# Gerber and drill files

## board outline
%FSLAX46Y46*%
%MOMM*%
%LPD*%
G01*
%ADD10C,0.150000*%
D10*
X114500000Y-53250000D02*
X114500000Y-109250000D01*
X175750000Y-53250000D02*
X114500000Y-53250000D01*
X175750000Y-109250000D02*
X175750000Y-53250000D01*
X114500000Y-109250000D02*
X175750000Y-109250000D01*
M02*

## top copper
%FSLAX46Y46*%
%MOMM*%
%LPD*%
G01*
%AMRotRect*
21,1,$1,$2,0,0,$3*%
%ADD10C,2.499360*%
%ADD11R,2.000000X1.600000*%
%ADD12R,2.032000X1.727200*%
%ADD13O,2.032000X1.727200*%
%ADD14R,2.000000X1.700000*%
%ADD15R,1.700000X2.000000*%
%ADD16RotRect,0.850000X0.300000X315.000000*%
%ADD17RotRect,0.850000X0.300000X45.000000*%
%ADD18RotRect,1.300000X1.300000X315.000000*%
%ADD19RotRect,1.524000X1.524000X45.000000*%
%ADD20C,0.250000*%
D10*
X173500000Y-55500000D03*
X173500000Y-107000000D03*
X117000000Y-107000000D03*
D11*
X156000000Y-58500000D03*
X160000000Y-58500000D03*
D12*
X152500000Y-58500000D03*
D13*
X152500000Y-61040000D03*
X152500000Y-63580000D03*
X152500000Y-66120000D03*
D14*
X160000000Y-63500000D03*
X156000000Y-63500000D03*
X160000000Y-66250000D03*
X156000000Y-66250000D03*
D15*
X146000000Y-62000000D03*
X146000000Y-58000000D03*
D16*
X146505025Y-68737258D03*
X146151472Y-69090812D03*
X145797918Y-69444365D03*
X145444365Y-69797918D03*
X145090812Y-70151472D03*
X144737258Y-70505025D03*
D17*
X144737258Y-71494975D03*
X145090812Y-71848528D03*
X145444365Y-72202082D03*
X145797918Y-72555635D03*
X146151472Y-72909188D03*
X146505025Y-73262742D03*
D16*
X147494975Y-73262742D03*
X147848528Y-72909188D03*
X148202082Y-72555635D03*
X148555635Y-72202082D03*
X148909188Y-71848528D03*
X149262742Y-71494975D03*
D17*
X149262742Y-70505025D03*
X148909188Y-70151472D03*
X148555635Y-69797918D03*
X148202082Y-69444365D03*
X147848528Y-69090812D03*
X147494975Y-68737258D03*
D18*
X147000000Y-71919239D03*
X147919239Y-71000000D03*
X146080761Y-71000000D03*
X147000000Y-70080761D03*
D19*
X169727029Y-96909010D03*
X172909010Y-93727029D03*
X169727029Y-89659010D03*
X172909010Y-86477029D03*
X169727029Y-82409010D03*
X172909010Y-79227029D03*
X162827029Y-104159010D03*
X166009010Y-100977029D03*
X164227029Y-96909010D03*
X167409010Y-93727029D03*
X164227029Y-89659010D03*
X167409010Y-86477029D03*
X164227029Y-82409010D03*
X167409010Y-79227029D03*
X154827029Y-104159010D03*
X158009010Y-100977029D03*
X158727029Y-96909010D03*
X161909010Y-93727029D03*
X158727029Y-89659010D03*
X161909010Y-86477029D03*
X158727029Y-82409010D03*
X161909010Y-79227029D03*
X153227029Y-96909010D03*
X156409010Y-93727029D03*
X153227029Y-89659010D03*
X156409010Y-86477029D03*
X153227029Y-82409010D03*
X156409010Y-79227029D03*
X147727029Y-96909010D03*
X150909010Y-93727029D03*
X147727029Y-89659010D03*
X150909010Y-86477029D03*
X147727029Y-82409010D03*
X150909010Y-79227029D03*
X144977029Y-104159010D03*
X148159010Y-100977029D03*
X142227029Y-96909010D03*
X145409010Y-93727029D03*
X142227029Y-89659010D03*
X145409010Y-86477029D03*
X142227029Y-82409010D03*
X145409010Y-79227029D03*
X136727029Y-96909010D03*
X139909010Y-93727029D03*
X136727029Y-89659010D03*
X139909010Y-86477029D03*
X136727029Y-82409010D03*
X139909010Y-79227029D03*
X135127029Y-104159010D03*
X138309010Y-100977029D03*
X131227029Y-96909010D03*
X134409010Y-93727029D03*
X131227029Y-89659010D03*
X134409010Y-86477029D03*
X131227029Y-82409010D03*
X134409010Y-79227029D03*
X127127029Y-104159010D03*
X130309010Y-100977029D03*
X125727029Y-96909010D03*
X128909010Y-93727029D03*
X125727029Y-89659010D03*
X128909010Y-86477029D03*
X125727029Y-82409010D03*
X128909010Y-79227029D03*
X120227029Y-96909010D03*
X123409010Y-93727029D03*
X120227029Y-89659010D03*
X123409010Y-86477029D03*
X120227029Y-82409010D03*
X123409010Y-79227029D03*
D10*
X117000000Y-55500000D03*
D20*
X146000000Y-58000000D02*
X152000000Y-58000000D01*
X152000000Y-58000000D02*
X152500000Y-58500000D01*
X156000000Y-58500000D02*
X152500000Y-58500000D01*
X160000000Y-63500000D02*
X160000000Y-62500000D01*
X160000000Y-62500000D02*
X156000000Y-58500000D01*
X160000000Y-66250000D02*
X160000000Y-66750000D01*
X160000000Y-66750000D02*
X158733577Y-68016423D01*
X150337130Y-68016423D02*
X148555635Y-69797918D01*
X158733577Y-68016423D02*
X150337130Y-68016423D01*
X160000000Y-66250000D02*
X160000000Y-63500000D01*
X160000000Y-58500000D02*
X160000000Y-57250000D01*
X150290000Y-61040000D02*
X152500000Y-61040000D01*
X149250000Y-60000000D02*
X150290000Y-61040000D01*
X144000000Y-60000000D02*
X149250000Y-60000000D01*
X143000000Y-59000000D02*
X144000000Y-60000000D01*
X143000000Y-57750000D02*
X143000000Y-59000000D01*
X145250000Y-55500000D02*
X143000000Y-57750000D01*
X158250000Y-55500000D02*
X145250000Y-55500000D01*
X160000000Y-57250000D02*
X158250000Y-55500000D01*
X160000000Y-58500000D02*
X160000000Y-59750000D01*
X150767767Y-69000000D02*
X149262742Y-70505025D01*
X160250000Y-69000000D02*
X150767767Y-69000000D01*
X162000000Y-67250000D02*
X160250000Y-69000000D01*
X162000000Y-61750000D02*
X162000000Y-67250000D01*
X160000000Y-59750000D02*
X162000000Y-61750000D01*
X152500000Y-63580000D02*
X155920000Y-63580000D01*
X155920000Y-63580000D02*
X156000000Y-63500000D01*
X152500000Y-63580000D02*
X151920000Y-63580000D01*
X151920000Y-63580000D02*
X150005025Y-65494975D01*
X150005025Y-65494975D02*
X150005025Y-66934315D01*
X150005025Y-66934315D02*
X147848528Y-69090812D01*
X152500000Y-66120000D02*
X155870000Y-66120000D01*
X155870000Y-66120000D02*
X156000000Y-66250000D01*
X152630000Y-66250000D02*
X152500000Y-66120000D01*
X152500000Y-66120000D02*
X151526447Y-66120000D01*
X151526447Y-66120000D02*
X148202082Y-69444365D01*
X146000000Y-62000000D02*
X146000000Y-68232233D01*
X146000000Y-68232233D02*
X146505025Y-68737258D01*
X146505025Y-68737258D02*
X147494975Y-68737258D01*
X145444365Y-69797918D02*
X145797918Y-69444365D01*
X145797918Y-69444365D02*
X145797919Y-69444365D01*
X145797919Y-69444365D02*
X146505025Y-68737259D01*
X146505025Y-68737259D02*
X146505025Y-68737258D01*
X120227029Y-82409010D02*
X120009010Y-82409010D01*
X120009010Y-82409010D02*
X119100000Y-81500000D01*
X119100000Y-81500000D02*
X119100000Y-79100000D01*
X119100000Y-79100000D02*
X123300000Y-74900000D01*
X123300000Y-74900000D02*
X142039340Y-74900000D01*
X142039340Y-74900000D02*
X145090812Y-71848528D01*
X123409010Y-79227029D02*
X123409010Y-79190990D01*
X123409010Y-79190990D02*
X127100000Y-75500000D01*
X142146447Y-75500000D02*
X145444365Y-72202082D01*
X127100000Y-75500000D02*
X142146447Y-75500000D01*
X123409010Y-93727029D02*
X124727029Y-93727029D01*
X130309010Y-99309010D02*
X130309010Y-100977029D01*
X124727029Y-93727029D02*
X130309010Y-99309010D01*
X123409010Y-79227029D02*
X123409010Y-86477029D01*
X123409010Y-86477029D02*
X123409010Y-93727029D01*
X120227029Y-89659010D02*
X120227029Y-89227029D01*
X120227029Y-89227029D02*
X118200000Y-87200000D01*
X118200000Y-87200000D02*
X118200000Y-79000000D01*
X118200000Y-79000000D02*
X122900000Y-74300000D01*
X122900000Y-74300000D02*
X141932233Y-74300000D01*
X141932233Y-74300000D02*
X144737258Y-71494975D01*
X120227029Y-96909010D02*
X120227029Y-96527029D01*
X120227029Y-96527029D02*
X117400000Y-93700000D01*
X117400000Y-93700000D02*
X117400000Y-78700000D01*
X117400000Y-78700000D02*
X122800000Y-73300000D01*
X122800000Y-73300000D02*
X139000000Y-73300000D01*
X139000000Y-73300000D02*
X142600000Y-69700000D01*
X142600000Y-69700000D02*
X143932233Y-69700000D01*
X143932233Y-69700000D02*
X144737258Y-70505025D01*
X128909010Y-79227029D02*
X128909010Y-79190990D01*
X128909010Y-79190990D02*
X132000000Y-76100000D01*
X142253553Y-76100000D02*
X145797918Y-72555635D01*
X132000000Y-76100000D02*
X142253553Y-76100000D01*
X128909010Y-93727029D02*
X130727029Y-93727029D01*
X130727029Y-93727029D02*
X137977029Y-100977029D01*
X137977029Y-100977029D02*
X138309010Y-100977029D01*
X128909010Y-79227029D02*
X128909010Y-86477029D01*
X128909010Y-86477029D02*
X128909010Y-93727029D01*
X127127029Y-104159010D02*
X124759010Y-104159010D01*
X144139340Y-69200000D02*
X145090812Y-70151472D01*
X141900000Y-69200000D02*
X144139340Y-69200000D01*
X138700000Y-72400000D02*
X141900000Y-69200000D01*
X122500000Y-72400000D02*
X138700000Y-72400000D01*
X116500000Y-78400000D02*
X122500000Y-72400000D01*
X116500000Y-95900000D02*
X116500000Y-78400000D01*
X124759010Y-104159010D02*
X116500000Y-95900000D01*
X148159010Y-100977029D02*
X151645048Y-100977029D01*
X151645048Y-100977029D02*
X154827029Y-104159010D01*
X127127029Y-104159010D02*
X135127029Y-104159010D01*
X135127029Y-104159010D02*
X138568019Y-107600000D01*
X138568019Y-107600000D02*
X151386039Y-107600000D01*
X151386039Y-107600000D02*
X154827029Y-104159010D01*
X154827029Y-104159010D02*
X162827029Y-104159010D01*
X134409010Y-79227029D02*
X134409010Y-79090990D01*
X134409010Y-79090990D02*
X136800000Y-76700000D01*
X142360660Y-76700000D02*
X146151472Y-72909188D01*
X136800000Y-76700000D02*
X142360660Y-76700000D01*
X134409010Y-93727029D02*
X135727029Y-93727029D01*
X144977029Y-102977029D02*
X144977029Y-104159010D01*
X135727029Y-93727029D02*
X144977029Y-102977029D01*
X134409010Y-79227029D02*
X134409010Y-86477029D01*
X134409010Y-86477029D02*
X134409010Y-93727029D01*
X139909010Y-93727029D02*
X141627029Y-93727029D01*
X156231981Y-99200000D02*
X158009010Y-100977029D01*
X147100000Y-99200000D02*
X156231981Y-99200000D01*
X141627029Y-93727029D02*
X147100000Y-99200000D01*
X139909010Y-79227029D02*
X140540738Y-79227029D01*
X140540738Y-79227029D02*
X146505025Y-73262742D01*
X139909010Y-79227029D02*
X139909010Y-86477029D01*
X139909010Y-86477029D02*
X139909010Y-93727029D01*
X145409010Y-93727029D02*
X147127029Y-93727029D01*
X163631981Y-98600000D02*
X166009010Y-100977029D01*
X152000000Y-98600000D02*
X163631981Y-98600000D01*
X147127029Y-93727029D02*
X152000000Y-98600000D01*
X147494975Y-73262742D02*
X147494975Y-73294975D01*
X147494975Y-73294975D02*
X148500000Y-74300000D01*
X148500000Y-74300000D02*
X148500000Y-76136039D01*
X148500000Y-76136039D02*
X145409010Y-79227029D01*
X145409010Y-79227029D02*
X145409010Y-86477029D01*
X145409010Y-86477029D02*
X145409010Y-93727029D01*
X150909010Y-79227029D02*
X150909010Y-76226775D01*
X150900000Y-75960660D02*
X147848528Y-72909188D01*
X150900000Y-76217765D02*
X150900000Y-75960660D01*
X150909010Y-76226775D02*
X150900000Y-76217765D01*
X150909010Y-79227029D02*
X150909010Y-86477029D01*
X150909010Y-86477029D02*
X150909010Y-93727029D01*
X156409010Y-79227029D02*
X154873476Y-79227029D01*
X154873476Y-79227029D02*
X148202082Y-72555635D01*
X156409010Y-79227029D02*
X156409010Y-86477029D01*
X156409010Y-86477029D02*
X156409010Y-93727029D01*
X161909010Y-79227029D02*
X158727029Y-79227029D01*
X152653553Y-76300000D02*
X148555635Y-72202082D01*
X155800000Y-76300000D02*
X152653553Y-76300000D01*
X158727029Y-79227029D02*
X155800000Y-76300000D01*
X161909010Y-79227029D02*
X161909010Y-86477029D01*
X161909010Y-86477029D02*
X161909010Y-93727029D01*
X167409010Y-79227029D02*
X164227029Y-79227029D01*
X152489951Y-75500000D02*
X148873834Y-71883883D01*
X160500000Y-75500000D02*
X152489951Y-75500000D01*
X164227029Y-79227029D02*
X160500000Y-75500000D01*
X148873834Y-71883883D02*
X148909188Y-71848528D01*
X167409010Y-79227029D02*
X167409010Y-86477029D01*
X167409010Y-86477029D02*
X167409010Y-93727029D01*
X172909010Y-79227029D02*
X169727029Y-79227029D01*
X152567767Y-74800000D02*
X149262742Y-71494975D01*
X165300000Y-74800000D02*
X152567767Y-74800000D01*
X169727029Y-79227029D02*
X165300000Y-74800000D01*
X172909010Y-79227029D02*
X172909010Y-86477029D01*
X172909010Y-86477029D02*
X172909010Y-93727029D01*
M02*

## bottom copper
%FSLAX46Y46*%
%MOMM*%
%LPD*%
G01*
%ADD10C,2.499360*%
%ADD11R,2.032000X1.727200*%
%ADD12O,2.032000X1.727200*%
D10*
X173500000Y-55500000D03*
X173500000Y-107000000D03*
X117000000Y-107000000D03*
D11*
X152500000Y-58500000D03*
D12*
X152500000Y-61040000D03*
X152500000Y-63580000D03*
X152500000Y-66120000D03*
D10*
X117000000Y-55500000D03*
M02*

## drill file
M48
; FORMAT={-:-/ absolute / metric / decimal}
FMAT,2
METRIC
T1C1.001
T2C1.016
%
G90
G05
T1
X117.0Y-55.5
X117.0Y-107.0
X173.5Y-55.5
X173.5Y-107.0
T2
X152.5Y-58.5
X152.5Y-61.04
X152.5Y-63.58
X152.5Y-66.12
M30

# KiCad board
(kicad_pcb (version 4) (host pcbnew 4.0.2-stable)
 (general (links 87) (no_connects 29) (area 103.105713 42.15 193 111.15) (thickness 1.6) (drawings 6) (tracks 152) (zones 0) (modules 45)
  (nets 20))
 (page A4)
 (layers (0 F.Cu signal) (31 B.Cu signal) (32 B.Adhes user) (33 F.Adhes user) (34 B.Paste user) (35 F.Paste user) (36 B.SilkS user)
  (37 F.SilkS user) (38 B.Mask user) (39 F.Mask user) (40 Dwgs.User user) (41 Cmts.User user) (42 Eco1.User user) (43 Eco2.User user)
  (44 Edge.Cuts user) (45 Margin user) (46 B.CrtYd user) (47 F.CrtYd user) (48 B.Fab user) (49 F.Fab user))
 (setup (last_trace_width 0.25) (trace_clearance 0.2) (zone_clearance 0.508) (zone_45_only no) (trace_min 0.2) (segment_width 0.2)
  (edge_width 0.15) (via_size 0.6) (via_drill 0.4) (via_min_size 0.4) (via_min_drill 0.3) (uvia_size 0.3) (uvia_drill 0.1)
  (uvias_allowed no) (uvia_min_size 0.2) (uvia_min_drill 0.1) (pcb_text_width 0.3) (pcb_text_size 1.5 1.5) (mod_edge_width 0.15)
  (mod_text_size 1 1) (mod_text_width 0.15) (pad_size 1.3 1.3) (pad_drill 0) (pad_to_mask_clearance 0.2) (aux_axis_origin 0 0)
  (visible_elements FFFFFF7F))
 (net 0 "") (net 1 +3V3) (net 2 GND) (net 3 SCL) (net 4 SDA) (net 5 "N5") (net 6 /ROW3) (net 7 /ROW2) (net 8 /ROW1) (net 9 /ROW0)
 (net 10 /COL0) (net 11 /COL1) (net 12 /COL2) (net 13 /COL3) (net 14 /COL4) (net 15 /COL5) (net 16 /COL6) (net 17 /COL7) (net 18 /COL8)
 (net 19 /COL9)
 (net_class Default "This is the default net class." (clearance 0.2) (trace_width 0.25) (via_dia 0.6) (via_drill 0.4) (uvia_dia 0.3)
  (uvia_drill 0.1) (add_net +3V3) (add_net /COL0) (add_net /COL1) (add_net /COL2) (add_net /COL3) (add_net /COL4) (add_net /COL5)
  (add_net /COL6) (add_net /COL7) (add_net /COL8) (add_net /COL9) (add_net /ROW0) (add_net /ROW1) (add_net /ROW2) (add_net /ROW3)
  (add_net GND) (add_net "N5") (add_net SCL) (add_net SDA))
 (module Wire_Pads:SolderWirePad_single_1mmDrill (layer F.Cu) (at 173.5 55.5)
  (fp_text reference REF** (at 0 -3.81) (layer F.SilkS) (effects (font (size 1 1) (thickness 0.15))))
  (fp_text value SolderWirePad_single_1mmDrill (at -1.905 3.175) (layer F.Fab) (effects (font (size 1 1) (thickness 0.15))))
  (pad 1 thru_hole circle (at 0 0) (size 2.49936 2.49936) (drill 1.00076) (layers *.Cu *.Mask F.SilkS)))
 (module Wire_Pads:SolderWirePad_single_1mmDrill (layer F.Cu) (at 173.5 107)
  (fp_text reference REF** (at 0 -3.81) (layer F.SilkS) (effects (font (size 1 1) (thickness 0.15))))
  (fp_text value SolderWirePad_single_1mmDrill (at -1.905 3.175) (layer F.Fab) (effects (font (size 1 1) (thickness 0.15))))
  (pad 1 thru_hole circle (at 0 0) (size 2.49936 2.49936) (drill 1.00076) (layers *.Cu *.Mask F.SilkS)))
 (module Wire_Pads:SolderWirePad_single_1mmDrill (layer F.Cu) (at 117 107)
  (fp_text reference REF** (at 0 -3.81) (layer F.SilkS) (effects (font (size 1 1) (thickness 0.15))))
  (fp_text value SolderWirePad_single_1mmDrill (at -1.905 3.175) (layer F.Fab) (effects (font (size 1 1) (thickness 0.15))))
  (pad 1 thru_hole circle (at 0 0) (size 2.49936 2.49936) (drill 1.00076) (layers *.Cu *.Mask F.SilkS)))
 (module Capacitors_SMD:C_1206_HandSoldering (layer F.Cu) (at 158 58.5)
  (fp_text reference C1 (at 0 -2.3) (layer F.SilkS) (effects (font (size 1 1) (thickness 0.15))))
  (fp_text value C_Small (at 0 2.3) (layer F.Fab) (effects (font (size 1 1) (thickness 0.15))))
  (pad 1 smd rect (at -2 0) (size 2 1.6) (layers F.Cu F.Paste F.Mask) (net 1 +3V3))
  (pad 2 smd rect (at 2 0) (size 2 1.6) (layers F.Cu F.Paste F.Mask) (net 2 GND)))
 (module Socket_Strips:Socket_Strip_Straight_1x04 (layer F.Cu) (at 152.5 58.5 270)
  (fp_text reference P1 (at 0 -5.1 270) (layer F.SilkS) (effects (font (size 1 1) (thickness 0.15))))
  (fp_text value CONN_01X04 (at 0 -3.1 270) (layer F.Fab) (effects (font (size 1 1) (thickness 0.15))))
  (pad 1 thru_hole rect (at 0 0 270) (size 1.7272 2.032) (drill 1.016) (layers *.Cu *.Mask F.SilkS) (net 1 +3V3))
  (pad 2 thru_hole oval (at 2.54 0 270) (size 1.7272 2.032) (drill 1.016) (layers *.Cu *.Mask F.SilkS) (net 2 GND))
  (pad 3 thru_hole oval (at 5.08 0 270) (size 1.7272 2.032) (drill 1.016) (layers *.Cu *.Mask F.SilkS) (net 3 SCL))
  (pad 4 thru_hole oval (at 7.62 0 270) (size 1.7272 2.032) (drill 1.016) (layers *.Cu *.Mask F.SilkS) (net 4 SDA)))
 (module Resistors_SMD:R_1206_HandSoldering (layer F.Cu) (at 158 63.5 180)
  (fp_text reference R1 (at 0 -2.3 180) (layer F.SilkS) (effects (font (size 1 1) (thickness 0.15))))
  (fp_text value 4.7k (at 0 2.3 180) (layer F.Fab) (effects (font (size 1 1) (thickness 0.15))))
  (pad 1 smd rect (at -2 0 180) (size 2 1.7) (layers F.Cu F.Paste F.Mask) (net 1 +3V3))
  (pad 2 smd rect (at 2 0 180) (size 2 1.7) (layers F.Cu F.Paste F.Mask) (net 3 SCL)))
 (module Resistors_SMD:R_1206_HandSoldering (layer F.Cu) (at 158 66.25 180)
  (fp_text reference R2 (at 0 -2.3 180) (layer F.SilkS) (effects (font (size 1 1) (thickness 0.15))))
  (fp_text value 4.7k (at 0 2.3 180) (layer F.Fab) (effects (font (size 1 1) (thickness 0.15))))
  (pad 1 smd rect (at -2 0 180) (size 2 1.7) (layers F.Cu F.Paste F.Mask) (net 1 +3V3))
  (pad 2 smd rect (at 2 0 180) (size 2 1.7) (layers F.Cu F.Paste F.Mask) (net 4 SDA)))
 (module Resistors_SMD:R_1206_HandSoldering (layer F.Cu) (at 146 60 90)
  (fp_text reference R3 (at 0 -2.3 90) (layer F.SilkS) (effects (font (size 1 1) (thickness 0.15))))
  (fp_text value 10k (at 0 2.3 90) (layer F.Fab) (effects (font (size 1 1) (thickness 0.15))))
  (pad 1 smd rect (at -2 0 90) (size 2 1.7) (layers F.Cu F.Paste F.Mask) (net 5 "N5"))
  (pad 2 smd rect (at 2 0 90) (size 2 1.7) (layers F.Cu F.Paste F.Mask) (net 1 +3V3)))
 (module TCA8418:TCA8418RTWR (layer F.Cu) (at 147 71 315)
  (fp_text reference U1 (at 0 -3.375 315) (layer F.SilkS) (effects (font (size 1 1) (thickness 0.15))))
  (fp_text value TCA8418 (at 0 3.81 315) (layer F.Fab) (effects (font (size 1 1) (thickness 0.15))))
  (pad 1 smd rect (at -1.95 -1.25 315) (size 0.85 0.3) (layers F.Cu F.Paste F.Mask) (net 5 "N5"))
  (pad 2 smd rect (at -1.95 -0.75 315) (size 0.85 0.3) (layers F.Cu F.Paste F.Mask) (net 5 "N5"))
  (pad 3 smd rect (at -1.95 -0.25 315) (size 0.85 0.3) (layers F.Cu F.Paste F.Mask) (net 5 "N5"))
  (pad 4 smd rect (at -1.95 0.25 315) (size 0.85 0.3) (layers F.Cu F.Paste F.Mask) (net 5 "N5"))
  (pad 5 smd rect (at -1.95 0.75 315) (size 0.85 0.3) (layers F.Cu F.Paste F.Mask) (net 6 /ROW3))
  (pad 6 smd rect (at -1.95 1.25 315) (size 0.85 0.3) (layers F.Cu F.Paste F.Mask) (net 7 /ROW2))
  (pad 7 smd rect (at -1.25 1.95 45) (size 0.85 0.3) (layers F.Cu F.Paste F.Mask) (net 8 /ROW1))
  (pad 8 smd rect (at -0.75 1.95 45) (size 0.85 0.3) (layers F.Cu F.Paste F.Mask) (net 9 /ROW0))
  (pad 9 smd rect (at -0.25 1.95 45) (size 0.85 0.3) (layers F.Cu F.Paste F.Mask) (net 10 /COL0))
  (pad 10 smd rect (at 0.25 1.95 45) (size 0.85 0.3) (layers F.Cu F.Paste F.Mask) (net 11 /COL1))
  (pad 11 smd rect (at 0.75 1.95 45) (size 0.85 0.3) (layers F.Cu F.Paste F.Mask) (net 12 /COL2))
  (pad 12 smd rect (at 1.25 1.95 45) (size 0.85 0.3) (layers F.Cu F.Paste F.Mask) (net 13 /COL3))
  (pad 13 smd rect (at 1.95 1.25 315) (size 0.85 0.3) (layers F.Cu F.Paste F.Mask) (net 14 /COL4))
  (pad 14 smd rect (at 1.95 0.75 315) (size 0.85 0.3) (layers F.Cu F.Paste F.Mask) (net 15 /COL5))
  (pad 15 smd rect (at 1.95 0.25 315) (size 0.85 0.3) (layers F.Cu F.Paste F.Mask) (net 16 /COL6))
  (pad 16 smd rect (at 1.95 -0.25 315) (size 0.85 0.3) (layers F.Cu F.Paste F.Mask) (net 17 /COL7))
  (pad 17 smd rect (at 1.95 -0.75 315) (size 0.85 0.3) (layers F.Cu F.Paste F.Mask) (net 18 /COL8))
  (pad 18 smd rect (at 1.95 -1.25 315) (size 0.85 0.3) (layers F.Cu F.Paste F.Mask) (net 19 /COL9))
  (pad 19 smd rect (at 1.25 -1.95 45) (size 0.85 0.3) (layers F.Cu F.Paste F.Mask) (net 2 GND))
  (pad 20 smd rect (at 0.75 -1.95 45) (size 0.85 0.3) (layers F.Cu F.Paste F.Mask) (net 5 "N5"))
  (pad 21 smd rect (at 0.25 -1.95 45) (size 0.85 0.3) (layers F.Cu F.Paste F.Mask) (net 1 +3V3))
  (pad 22 smd rect (at -0.25 -1.95 45) (size 0.85 0.3) (layers F.Cu F.Paste F.Mask) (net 4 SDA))
  (pad 23 smd rect (at -0.75 -1.95 45) (size 0.85 0.3) (layers F.Cu F.Paste F.Mask) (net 3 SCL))
  (pad 24 smd rect (at -1.25 -1.95 45) (size 0.85 0.3) (layers F.Cu F.Paste F.Mask) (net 5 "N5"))
  (pad 25 smd rect (at 0.65 0.65 315) (size 1.3 1.3) (layers F.Cu F.Paste F.Mask) (solder_paste_margin_ratio -0.2))
  (pad 25 smd rect (at 0.65 -0.65 315) (size 1.3 1.3) (layers F.Cu F.Paste F.Mask) (solder_paste_margin_ratio -0.2))
  (pad 25 smd rect (at -0.65 0.65 315) (size 1.3 1.3) (layers F.Cu F.Paste F.Mask) (solder_paste_margin_ratio -0.2))
  (pad 25 smd rect (at -0.65 -0.65 315) (size 1.3 1.3) (layers F.Cu F.Paste F.Mask) (solder_paste_margin_ratio -0.2)))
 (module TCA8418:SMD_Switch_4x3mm (layer F.Cu) (at 174.5 98.5 45)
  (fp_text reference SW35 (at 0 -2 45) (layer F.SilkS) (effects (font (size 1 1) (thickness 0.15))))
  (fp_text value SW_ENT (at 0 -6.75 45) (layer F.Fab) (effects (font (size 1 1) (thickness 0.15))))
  (pad 1 smd rect (at -2.25 -4.5 45) (size 1.524 1.524) (layers F.Cu F.Paste F.Mask) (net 7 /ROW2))
  (pad 2 smd rect (at 2.25 -4.5 45) (size 1.524 1.524) (layers F.Cu F.Paste F.Mask) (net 19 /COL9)))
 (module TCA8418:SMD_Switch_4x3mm (layer F.Cu) (at 174.5 91.25 45)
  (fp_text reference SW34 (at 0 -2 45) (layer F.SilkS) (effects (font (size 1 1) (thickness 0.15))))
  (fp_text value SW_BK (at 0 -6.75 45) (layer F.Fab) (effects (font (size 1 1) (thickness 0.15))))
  (pad 1 smd rect (at -2.25 -4.5 45) (size 1.524 1.524) (layers F.Cu F.Paste F.Mask) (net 8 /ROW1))
  (pad 2 smd rect (at 2.25 -4.5 45) (size 1.524 1.524) (layers F.Cu F.Paste F.Mask) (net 19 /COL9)))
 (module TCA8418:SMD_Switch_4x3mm (layer F.Cu) (at 174.5 84 45)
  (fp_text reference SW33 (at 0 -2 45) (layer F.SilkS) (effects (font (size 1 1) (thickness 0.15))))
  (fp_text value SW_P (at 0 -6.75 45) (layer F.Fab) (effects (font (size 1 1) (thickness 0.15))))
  (pad 1 smd rect (at -2.25 -4.5 45) (size 1.524 1.524) (layers F.Cu F.Paste F.Mask) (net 9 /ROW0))
  (pad 2 smd rect (at 2.25 -4.5 45) (size 1.524 1.524) (layers F.Cu F.Paste F.Mask) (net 19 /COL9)))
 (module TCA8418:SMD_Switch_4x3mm (layer F.Cu) (at 167.6 105.75 45)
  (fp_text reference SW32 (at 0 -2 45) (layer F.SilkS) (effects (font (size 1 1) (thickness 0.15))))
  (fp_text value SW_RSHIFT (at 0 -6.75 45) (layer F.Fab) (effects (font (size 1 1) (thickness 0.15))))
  (pad 1 smd rect (at -2.25 -4.5 45) (size 1.524 1.524) (layers F.Cu F.Paste F.Mask) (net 6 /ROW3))
  (pad 2 smd rect (at 2.25 -4.5 45) (size 1.524 1.524) (layers F.Cu F.Paste F.Mask) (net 14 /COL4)))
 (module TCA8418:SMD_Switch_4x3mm (layer F.Cu) (at 169 98.5 45)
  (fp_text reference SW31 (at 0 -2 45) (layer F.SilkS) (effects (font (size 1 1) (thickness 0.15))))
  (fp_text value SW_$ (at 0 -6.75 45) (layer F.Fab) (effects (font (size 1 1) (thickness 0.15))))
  (pad 1 smd rect (at -2.25 -4.5 45) (size 1.524 1.524) (layers F.Cu F.Paste F.Mask) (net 7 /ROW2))
  (pad 2 smd rect (at 2.25 -4.5 45) (size 1.524 1.524) (layers F.Cu F.Paste F.Mask) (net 18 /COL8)))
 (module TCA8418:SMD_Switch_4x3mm (layer F.Cu) (at 169 91.25 45)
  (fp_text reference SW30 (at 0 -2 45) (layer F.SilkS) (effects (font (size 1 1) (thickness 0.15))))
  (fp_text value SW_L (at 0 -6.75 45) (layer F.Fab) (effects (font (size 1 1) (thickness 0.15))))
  (pad 1 smd rect (at -2.25 -4.5 45) (size 1.524 1.524) (layers F.Cu F.Paste F.Mask) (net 8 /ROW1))
  (pad 2 smd rect (at 2.25 -4.5 45) (size 1.524 1.524) (layers F.Cu F.Paste F.Mask) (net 18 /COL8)))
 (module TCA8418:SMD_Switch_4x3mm (layer F.Cu) (at 169 84 45)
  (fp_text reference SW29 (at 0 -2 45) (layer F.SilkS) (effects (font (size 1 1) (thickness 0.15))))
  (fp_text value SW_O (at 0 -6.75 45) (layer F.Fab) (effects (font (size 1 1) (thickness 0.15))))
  (pad 1 smd rect (at -2.25 -4.5 45) (size 1.524 1.524) (layers F.Cu F.Paste F.Mask) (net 9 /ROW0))
  (pad 2 smd rect (at 2.25 -4.5 45) (size 1.524 1.524) (layers F.Cu F.Paste F.Mask) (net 18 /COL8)))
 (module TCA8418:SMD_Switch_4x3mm (layer F.Cu) (at 159.6 105.75 45)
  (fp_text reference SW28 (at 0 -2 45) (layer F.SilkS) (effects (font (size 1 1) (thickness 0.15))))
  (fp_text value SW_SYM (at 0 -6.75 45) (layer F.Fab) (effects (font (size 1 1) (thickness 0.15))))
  (pad 1 smd rect (at -2.25 -4.5 45) (size 1.524 1.524) (layers F.Cu F.Paste F.Mask) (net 6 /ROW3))
  (pad 2 smd rect (at 2.25 -4.5 45) (size 1.524 1.524) (layers F.Cu F.Paste F.Mask) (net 13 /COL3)))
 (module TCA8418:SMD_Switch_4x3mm (layer F.Cu) (at 163.5 98.5 45)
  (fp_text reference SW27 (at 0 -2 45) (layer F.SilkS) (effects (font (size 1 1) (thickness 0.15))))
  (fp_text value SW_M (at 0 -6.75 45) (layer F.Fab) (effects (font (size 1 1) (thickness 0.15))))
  (pad 1 smd rect (at -2.25 -4.5 45) (size 1.524 1.524) (layers F.Cu F.Paste F.Mask) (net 7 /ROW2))
  (pad 2 smd rect (at 2.25 -4.5 45) (size 1.524 1.524) (layers F.Cu F.Paste F.Mask) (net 17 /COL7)))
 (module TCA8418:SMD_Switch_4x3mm (layer F.Cu) (at 163.5 91.25 45)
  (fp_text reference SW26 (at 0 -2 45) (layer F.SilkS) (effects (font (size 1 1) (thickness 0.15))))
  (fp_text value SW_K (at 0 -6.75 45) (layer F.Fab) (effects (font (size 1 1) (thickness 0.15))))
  (pad 1 smd rect (at -2.25 -4.5 45) (size 1.524 1.524) (layers F.Cu F.Paste F.Mask) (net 8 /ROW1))
  (pad 2 smd rect (at 2.25 -4.5 45) (size 1.524 1.524) (layers F.Cu F.Paste F.Mask) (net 17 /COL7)))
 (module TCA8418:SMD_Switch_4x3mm (layer F.Cu) (at 163.5 84 45)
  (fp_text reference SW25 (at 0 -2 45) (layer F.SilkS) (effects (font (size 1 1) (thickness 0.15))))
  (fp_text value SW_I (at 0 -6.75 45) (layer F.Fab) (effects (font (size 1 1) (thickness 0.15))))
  (pad 1 smd rect (at -2.25 -4.5 45) (size 1.524 1.524) (layers F.Cu F.Paste F.Mask) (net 9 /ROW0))
  (pad 2 smd rect (at 2.25 -4.5 45) (size 1.524 1.524) (layers F.Cu F.Paste F.Mask) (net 17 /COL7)))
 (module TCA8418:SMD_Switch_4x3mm (layer F.Cu) (at 158 98.5 45)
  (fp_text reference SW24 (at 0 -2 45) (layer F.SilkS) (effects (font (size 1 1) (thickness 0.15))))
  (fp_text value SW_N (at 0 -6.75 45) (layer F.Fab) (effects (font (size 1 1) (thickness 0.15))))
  (pad 1 smd rect (at -2.25 -4.5 45) (size 1.524 1.524) (layers F.Cu F.Paste F.Mask) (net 7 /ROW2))
  (pad 2 smd rect (at 2.25 -4.5 45) (size 1.524 1.524) (layers F.Cu F.Paste F.Mask) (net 16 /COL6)))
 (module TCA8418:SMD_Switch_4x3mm (layer F.Cu) (at 158 91.25 45)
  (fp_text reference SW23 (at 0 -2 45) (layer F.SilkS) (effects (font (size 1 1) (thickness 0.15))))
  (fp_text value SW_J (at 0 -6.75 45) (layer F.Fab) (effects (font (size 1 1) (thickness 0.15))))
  (pad 1 smd rect (at -2.25 -4.5 45) (size 1.524 1.524) (layers F.Cu F.Paste F.Mask) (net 8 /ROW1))
  (pad 2 smd rect (at 2.25 -4.5 45) (size 1.524 1.524) (layers F.Cu F.Paste F.Mask) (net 16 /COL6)))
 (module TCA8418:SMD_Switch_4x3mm (layer F.Cu) (at 158 84 45)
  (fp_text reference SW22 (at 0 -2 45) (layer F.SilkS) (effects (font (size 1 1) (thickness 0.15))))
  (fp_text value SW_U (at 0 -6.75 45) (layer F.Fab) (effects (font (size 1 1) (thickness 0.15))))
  (pad 1 smd rect (at -2.25 -4.5 45) (size 1.524 1.524) (layers F.Cu F.Paste F.Mask) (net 9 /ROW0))
  (pad 2 smd rect (at 2.25 -4.5 45) (size 1.524 1.524) (layers F.Cu F.Paste F.Mask) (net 16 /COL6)))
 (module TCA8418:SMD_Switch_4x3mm (layer F.Cu) (at 152.5 98.5 45)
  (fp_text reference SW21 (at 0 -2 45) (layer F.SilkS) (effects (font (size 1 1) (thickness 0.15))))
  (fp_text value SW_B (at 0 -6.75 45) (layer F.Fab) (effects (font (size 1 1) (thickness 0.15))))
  (pad 1 smd rect (at -2.25 -4.5 45) (size 1.524 1.524) (layers F.Cu F.Paste F.Mask) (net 7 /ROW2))
  (pad 2 smd rect (at 2.25 -4.5 45) (size 1.524 1.524) (layers F.Cu F.Paste F.Mask) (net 15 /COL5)))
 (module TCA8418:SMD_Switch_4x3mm (layer F.Cu) (at 152.5 91.25 45)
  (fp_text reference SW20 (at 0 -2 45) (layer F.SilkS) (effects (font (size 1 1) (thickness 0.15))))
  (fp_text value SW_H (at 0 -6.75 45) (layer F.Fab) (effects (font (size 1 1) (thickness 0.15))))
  (pad 1 smd rect (at -2.25 -4.5 45) (size 1.524 1.524) (layers F.Cu F.Paste F.Mask) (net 8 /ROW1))
  (pad 2 smd rect (at 2.25 -4.5 45) (size 1.524 1.524) (layers F.Cu F.Paste F.Mask) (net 15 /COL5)))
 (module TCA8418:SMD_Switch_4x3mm (layer F.Cu) (at 152.5 84 45)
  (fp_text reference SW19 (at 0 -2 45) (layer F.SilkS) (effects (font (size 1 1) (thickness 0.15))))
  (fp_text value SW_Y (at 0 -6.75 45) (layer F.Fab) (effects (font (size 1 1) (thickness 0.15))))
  (pad 1 smd rect (at -2.25 -4.5 45) (size 1.524 1.524) (layers F.Cu F.Paste F.Mask) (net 9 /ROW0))
  (pad 2 smd rect (at 2.25 -4.5 45) (size 1.524 1.524) (layers F.Cu F.Paste F.Mask) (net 15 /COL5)))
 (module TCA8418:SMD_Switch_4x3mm (layer F.Cu) (at 149.75 105.75 45)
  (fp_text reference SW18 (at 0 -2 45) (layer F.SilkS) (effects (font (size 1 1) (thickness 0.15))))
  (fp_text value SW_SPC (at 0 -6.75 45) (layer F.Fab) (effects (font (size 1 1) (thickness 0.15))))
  (pad 1 smd rect (at -2.25 -4.5 45) (size 1.524 1.524) (layers F.Cu F.Paste F.Mask) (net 12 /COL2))
  (pad 2 smd rect (at 2.25 -4.5 45) (size 1.524 1.524) (layers F.Cu F.Paste F.Mask) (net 6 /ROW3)))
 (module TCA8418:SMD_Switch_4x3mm (layer F.Cu) (at 147 98.5 45)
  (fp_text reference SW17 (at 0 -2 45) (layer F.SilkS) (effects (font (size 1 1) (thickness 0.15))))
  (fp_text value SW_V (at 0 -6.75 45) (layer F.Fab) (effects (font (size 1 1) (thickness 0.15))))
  (pad 1 smd rect (at -2.25 -4.5 45) (size 1.524 1.524) (layers F.Cu F.Paste F.Mask) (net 7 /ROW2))
  (pad 2 smd rect (at 2.25 -4.5 45) (size 1.524 1.524) (layers F.Cu F.Paste F.Mask) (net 14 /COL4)))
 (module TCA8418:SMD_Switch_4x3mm (layer F.Cu) (at 147 91.25 45)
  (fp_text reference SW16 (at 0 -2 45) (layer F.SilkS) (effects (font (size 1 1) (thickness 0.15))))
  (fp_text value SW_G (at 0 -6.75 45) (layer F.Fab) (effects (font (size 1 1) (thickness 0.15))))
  (pad 1 smd rect (at -2.25 -4.5 45) (size 1.524 1.524) (layers F.Cu F.Paste F.Mask) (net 8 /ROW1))
  (pad 2 smd rect (at 2.25 -4.5 45) (size 1.524 1.524) (layers F.Cu F.Paste F.Mask) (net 14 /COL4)))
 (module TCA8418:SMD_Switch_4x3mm (layer F.Cu) (at 147 84 45)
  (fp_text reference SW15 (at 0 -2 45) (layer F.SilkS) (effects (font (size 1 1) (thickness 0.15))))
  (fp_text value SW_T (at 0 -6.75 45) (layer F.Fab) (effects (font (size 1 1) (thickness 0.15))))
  (pad 1 smd rect (at -2.25 -4.5 45) (size 1.524 1.524) (layers F.Cu F.Paste F.Mask) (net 9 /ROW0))
  (pad 2 smd rect (at 2.25 -4.5 45) (size 1.524 1.524) (layers F.Cu F.Paste F.Mask) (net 14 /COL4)))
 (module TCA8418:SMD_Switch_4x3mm (layer F.Cu) (at 141.5 98.5 45)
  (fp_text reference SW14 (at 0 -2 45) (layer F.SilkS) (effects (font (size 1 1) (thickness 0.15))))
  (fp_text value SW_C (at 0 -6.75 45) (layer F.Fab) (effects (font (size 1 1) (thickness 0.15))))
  (pad 1 smd rect (at -2.25 -4.5 45) (size 1.524 1.524) (layers F.Cu F.Paste F.Mask) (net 7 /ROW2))
  (pad 2 smd rect (at 2.25 -4.5 45) (size 1.524 1.524) (layers F.Cu F.Paste F.Mask) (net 13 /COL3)))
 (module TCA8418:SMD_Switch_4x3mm (layer F.Cu) (at 141.5 91.25 45)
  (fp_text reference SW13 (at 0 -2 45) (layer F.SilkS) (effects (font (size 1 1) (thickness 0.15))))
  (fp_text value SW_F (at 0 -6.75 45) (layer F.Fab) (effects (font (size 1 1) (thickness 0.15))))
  (pad 1 smd rect (at -2.25 -4.5 45) (size 1.524 1.524) (layers F.Cu F.Paste F.Mask) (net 8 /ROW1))
  (pad 2 smd rect (at 2.25 -4.5 45) (size 1.524 1.524) (layers F.Cu F.Paste F.Mask) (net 13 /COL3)))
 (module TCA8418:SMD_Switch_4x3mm (layer F.Cu) (at 141.5 84 45)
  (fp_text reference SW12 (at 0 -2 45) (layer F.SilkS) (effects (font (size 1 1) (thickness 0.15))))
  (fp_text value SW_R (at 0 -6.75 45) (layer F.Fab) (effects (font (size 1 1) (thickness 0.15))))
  (pad 1 smd rect (at -2.25 -4.5 45) (size 1.524 1.524) (layers F.Cu F.Paste F.Mask) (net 9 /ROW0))
  (pad 2 smd rect (at 2.25 -4.5 45) (size 1.524 1.524) (layers F.Cu F.Paste F.Mask) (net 13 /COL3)))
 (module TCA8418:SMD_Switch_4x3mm (layer F.Cu) (at 139.9 105.75 45)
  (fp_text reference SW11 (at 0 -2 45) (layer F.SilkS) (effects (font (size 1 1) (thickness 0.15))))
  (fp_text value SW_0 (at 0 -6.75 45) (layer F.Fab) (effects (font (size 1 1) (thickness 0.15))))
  (pad 1 smd rect (at -2.25 -4.5 45) (size 1.524 1.524) (layers F.Cu F.Paste F.Mask) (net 6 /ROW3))
  (pad 2 smd rect (at 2.25 -4.5 45) (size 1.524 1.524) (layers F.Cu F.Paste F.Mask) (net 11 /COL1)))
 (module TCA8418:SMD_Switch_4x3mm (layer F.Cu) (at 136 98.5 45)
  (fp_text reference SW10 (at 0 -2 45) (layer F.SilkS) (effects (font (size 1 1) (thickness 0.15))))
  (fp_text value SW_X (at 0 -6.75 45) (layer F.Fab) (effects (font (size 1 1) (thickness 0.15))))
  (pad 1 smd rect (at -2.25 -4.5 45) (size 1.524 1.524) (layers F.Cu F.Paste F.Mask) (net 7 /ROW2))
  (pad 2 smd rect (at 2.25 -4.5 45) (size 1.524 1.524) (layers F.Cu F.Paste F.Mask) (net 12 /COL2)))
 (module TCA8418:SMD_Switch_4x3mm (layer F.Cu) (at 136 91.25 45)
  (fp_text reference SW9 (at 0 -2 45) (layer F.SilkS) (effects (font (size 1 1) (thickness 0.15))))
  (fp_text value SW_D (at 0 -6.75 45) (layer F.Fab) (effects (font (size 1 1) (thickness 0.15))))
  (pad 1 smd rect (at -2.25 -4.5 45) (size 1.524 1.524) (layers F.Cu F.Paste F.Mask) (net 8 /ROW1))
  (pad 2 smd rect (at 2.25 -4.5 45) (size 1.524 1.524) (layers F.Cu F.Paste F.Mask) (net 12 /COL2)))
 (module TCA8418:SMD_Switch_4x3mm (layer F.Cu) (at 136 84 45)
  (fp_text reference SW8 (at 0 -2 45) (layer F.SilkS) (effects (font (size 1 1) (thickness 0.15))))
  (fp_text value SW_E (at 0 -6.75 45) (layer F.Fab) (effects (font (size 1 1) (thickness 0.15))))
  (pad 1 smd rect (at -2.25 -4.5 45) (size 1.524 1.524) (layers F.Cu F.Paste F.Mask) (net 9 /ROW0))
  (pad 2 smd rect (at 2.25 -4.5 45) (size 1.524 1.524) (layers F.Cu F.Paste F.Mask) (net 12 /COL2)))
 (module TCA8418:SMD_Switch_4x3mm (layer F.Cu) (at 131.9 105.75 45)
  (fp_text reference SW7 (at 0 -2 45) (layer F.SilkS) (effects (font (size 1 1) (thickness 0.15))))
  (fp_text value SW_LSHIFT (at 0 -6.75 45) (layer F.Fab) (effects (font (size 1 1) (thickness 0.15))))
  (pad 1 smd rect (at -2.25 -4.5 45) (size 1.524 1.524) (layers F.Cu F.Paste F.Mask) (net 6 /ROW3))
  (pad 2 smd rect (at 2.25 -4.5 45) (size 1.524 1.524) (layers F.Cu F.Paste F.Mask) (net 10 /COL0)))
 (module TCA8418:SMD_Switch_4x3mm (layer F.Cu) (at 130.5 98.5 45)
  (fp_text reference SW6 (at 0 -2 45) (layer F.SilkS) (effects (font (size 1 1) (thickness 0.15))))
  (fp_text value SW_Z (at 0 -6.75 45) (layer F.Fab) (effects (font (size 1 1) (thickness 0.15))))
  (pad 1 smd rect (at -2.25 -4.5 45) (size 1.524 1.524) (layers F.Cu F.Paste F.Mask) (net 7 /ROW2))
  (pad 2 smd rect (at 2.25 -4.5 45) (size 1.524 1.524) (layers F.Cu F.Paste F.Mask) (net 11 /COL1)))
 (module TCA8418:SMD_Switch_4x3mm (layer F.Cu) (at 130.5 91.25 45)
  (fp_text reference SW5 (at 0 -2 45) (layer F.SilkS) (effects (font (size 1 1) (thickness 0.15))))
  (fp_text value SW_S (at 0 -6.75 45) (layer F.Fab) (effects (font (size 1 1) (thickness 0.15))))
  (pad 1 smd rect (at -2.25 -4.5 45) (size 1.524 1.524) (layers F.Cu F.Paste F.Mask) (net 8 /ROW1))
  (pad 2 smd rect (at 2.25 -4.5 45) (size 1.524 1.524) (layers F.Cu F.Paste F.Mask) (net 11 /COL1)))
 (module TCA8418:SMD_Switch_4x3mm (layer F.Cu) (at 130.5 84 45)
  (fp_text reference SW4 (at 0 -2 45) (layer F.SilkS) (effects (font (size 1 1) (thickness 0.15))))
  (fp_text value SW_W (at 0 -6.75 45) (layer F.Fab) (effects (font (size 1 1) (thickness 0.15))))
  (pad 1 smd rect (at -2.25 -4.5 45) (size 1.524 1.524) (layers F.Cu F.Paste F.Mask) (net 9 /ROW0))
  (pad 2 smd rect (at 2.25 -4.5 45) (size 1.524 1.524) (layers F.Cu F.Paste F.Mask) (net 11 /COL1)))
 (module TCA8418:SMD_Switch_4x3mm (layer F.Cu) (at 125 98.5 45)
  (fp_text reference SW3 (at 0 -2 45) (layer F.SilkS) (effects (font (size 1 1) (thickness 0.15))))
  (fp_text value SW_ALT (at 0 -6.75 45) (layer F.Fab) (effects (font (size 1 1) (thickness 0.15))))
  (pad 1 smd rect (at -2.25 -4.5 45) (size 1.524 1.524) (layers F.Cu F.Paste F.Mask) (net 7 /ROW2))
  (pad 2 smd rect (at 2.25 -4.5 45) (size 1.524 1.524) (layers F.Cu F.Paste F.Mask) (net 10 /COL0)))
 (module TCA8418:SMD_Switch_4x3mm (layer F.Cu) (at 125 91.25 45)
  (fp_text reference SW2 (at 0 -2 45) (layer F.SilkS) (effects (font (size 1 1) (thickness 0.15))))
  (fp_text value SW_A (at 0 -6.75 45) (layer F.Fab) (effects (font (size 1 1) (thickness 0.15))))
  (pad 1 smd rect (at -2.25 -4.5 45) (size 1.524 1.524) (layers F.Cu F.Paste F.Mask) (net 8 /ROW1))
  (pad 2 smd rect (at 2.25 -4.5 45) (size 1.524 1.524) (layers F.Cu F.Paste F.Mask) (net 10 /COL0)))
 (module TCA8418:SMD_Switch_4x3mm (layer F.Cu) (at 125 84 45)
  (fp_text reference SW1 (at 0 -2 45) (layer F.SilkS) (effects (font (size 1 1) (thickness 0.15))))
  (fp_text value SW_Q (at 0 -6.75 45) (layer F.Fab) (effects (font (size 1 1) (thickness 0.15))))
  (pad 1 smd rect (at -2.25 -4.5 45) (size 1.524 1.524) (layers F.Cu F.Paste F.Mask) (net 9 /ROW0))
  (pad 2 smd rect (at 2.25 -4.5 45) (size 1.524 1.524) (layers F.Cu F.Paste F.Mask) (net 10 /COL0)))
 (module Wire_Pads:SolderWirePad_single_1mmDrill (layer F.Cu) (at 117 55.5)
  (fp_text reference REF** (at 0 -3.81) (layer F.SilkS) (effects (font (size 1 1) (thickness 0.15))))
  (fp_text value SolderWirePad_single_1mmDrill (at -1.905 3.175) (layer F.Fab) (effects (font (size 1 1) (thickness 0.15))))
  (pad 1 thru_hole circle (at 0 0) (size 2.49936 2.49936) (drill 1.00076) (layers *.Cu *.Mask F.SilkS)))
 (gr_line (start 114.5 53.25) (end 114.5 109.25) (angle 90) (layer Edge.Cuts) (width 0.15))
 (gr_line (start 175.75 53.25) (end 114.5 53.25) (angle 90) (layer Edge.Cuts) (width 0.15))
 (gr_line (start 175.75 109.25) (end 175.75 53.25) (angle 90) (layer Edge.Cuts) (width 0.15))
 (gr_line (start 114.5 109.25) (end 175.75 109.25) (angle 90) (layer Edge.Cuts) (width 0.15))
 (segment (start 146 58) (end 152 58) (width 0.25) (layer F.Cu) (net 1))
 (segment (start 152 58) (end 152.5 58.5) (width 0.25) (layer F.Cu) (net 1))
 (segment (start 156 58.5) (end 152.5 58.5) (width 0.25) (layer F.Cu) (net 1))
 (segment (start 160 63.5) (end 160 62.5) (width 0.25) (layer F.Cu) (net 1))
 (segment (start 160 62.5) (end 156 58.5) (width 0.25) (layer F.Cu) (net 1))
 (segment (start 160 66.25) (end 160 66.75) (width 0.25) (layer F.Cu) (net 1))
 (segment (start 160 66.75) (end 158.733577 68.016423) (width 0.25) (layer F.Cu) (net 1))
 (segment (start 150.33713 68.016423) (end 148.555635 69.797918) (width 0.25) (layer F.Cu) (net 1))
 (segment (start 158.733577 68.016423) (end 150.33713 68.016423) (width 0.25) (layer F.Cu) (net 1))
 (segment (start 160 66.25) (end 160 63.5) (width 0.25) (layer F.Cu) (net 1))
 (segment (start 160 58.5) (end 160 57.25) (width 0.25) (layer F.Cu) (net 2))
 (segment (start 150.29 61.04) (end 152.5 61.04) (width 0.25) (layer F.Cu) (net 2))
 (segment (start 149.25 60) (end 150.29 61.04) (width 0.25) (layer F.Cu) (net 2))
 (segment (start 144 60) (end 149.25 60) (width 0.25) (layer F.Cu) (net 2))
 (segment (start 143 59) (end 144 60) (width 0.25) (layer F.Cu) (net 2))
 (segment (start 143 57.75) (end 143 59) (width 0.25) (layer F.Cu) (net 2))
 (segment (start 145.25 55.5) (end 143 57.75) (width 0.25) (layer F.Cu) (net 2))
 (segment (start 158.25 55.5) (end 145.25 55.5) (width 0.25) (layer F.Cu) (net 2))
 (segment (start 160 57.25) (end 158.25 55.5) (width 0.25) (layer F.Cu) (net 2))
 (segment (start 160 58.5) (end 160 59.75) (width 0.25) (layer F.Cu) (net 2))
 (segment (start 150.767767 69) (end 149.262742 70.505025) (width 0.25) (layer F.Cu) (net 2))
 (segment (start 160.25 69) (end 150.767767 69) (width 0.25) (layer F.Cu) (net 2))
 (segment (start 162 67.25) (end 160.25 69) (width 0.25) (layer F.Cu) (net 2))
 (segment (start 162 61.75) (end 162 67.25) (width 0.25) (layer F.Cu) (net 2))
 (segment (start 160 59.75) (end 162 61.75) (width 0.25) (layer F.Cu) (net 2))
 (segment (start 152.5 63.58) (end 155.92 63.58) (width 0.25) (layer F.Cu) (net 3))
 (segment (start 155.92 63.58) (end 156 63.5) (width 0.25) (layer F.Cu) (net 3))
 (segment (start 152.5 63.58) (end 151.92 63.58) (width 0.25) (layer F.Cu) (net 3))
 (segment (start 151.92 63.58) (end 150.005025 65.494975) (width 0.25) (layer F.Cu) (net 3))
 (segment (start 150.005025 65.494975) (end 150.005025 66.934315) (width 0.25) (layer F.Cu) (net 3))
 (segment (start 150.005025 66.934315) (end 147.848528 69.090812) (width 0.25) (layer F.Cu) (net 3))
 (segment (start 152.5 66.12) (end 155.87 66.12) (width 0.25) (layer F.Cu) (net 4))
 (segment (start 155.87 66.12) (end 156 66.25) (width 0.25) (layer F.Cu) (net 4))
 (segment (start 152.63 66.25) (end 152.5 66.12) (width 0.25) (layer F.Cu) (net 4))
 (segment (start 152.5 66.12) (end 151.526447 66.12) (width 0.25) (layer F.Cu) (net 4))
 (segment (start 151.526447 66.12) (end 148.202082 69.444365) (width 0.25) (layer F.Cu) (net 4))
 (segment (start 146 62) (end 146 68.232233) (width 0.25) (layer F.Cu) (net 5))
 (segment (start 146 68.232233) (end 146.505025 68.737258) (width 0.25) (layer F.Cu) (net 5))
 (segment (start 146.505025 68.737258) (end 147.494975 68.737258) (width 0.25) (layer F.Cu) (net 5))
 (segment (start 145.444365 69.797918) (end 145.797918 69.444365) (width 0.25) (layer F.Cu) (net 5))
 (segment (start 145.797918 69.444365) (end 145.797919 69.444365) (width 0.25) (layer F.Cu) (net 5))
 (segment (start 145.797919 69.444365) (end 146.505025 68.737259) (width 0.25) (layer F.Cu) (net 5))
 (segment (start 146.505025 68.737259) (end 146.505025 68.737258) (width 0.25) (layer F.Cu) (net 5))
 (segment (start 120.227029 82.40901) (end 120.00901 82.40901) (width 0.25) (layer F.Cu) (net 9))
 (segment (start 120.00901 82.40901) (end 119.1 81.5) (width 0.25) (layer F.Cu) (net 9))
 (segment (start 119.1 81.5) (end 119.1 79.1) (width 0.25) (layer F.Cu) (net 9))
 (segment (start 119.1 79.1) (end 123.3 74.9) (width 0.25) (layer F.Cu) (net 9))
 (segment (start 123.3 74.9) (end 142.03934 74.9) (width 0.25) (layer F.Cu) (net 9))
 (segment (start 142.03934 74.9) (end 145.090812 71.848528) (width 0.25) (layer F.Cu) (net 9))
 (segment (start 123.40901 79.227029) (end 123.40901 79.19099) (width 0.25) (layer F.Cu) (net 10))
 (segment (start 123.40901 79.19099) (end 127.1 75.5) (width 0.25) (layer F.Cu) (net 10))
 (segment (start 142.146447 75.5) (end 145.444365 72.202082) (width 0.25) (layer F.Cu) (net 10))
 (segment (start 127.1 75.5) (end 142.146447 75.5) (width 0.25) (layer F.Cu) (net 10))
 (segment (start 123.40901 93.727029) (end 124.727029 93.727029) (width 0.25) (layer F.Cu) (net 10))
 (segment (start 130.30901 99.30901) (end 130.30901 100.977029) (width 0.25) (layer F.Cu) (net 10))
 (segment (start 124.727029 93.727029) (end 130.30901 99.30901) (width 0.25) (layer F.Cu) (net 10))
 (segment (start 123.40901 79.227029) (end 123.40901 86.477029) (width 0.25) (layer F.Cu) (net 10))
 (segment (start 123.40901 86.477029) (end 123.40901 93.727029) (width 0.25) (layer F.Cu) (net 10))
 (segment (start 120.227029 89.65901) (end 120.227029 89.227029) (width 0.25) (layer F.Cu) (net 8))
 (segment (start 120.227029 89.227029) (end 118.2 87.2) (width 0.25) (layer F.Cu) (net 8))
 (segment (start 118.2 87.2) (end 118.2 79) (width 0.25) (layer F.Cu) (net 8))
 (segment (start 118.2 79) (end 122.9 74.3) (width 0.25) (layer F.Cu) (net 8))
 (segment (start 122.9 74.3) (end 141.932233 74.3) (width 0.25) (layer F.Cu) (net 8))
 (segment (start 141.932233 74.3) (end 144.737258 71.494975) (width 0.25) (layer F.Cu) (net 8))
 (segment (start 120.227029 96.90901) (end 120.227029 96.527029) (width 0.25) (layer F.Cu) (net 7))
 (segment (start 120.227029 96.527029) (end 117.4 93.7) (width 0.25) (layer F.Cu) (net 7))
 (segment (start 117.4 93.7) (end 117.4 78.7) (width 0.25) (layer F.Cu) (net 7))
 (segment (start 117.4 78.7) (end 122.8 73.3) (width 0.25) (layer F.Cu) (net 7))
 (segment (start 122.8 73.3) (end 139 73.3) (width 0.25) (layer F.Cu) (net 7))
 (segment (start 139 73.3) (end 142.6 69.7) (width 0.25) (layer F.Cu) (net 7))
 (segment (start 142.6 69.7) (end 143.932233 69.7) (width 0.25) (layer F.Cu) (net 7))
 (segment (start 143.932233 69.7) (end 144.737258 70.505025) (width 0.25) (layer F.Cu) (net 7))
 (segment (start 128.90901 79.227029) (end 128.90901 79.19099) (width 0.25) (layer F.Cu) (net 11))
 (segment (start 128.90901 79.19099) (end 132 76.1) (width 0.25) (layer F.Cu) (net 11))
 (segment (start 142.253553 76.1) (end 145.797918 72.555635) (width 0.25) (layer F.Cu) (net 11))
 (segment (start 132 76.1) (end 142.253553 76.1) (width 0.25) (layer F.Cu) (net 11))
 (segment (start 128.90901 93.727029) (end 130.727029 93.727029) (width 0.25) (layer F.Cu) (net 11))
 (segment (start 130.727029 93.727029) (end 137.977029 100.977029) (width 0.25) (layer F.Cu) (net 11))
 (segment (start 137.977029 100.977029) (end 138.30901 100.977029) (width 0.25) (layer F.Cu) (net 11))
 (segment (start 128.90901 79.227029) (end 128.90901 86.477029) (width 0.25) (layer F.Cu) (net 11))
 (segment (start 128.90901 86.477029) (end 128.90901 93.727029) (width 0.25) (layer F.Cu) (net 11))
 (segment (start 127.127029 104.15901) (end 124.75901 104.15901) (width 0.25) (layer F.Cu) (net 6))
 (segment (start 144.13934 69.2) (end 145.090812 70.151472) (width 0.25) (layer F.Cu) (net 6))
 (segment (start 141.9 69.2) (end 144.13934 69.2) (width 0.25) (layer F.Cu) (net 6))
 (segment (start 138.7 72.4) (end 141.9 69.2) (width 0.25) (layer F.Cu) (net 6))
 (segment (start 122.5 72.4) (end 138.7 72.4) (width 0.25) (layer F.Cu) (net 6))
 (segment (start 116.5 78.4) (end 122.5 72.4) (width 0.25) (layer F.Cu) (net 6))
 (segment (start 116.5 95.9) (end 116.5 78.4) (width 0.25) (layer F.Cu) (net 6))
 (segment (start 124.75901 104.15901) (end 116.5 95.9) (width 0.25) (layer F.Cu) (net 6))
 (segment (start 148.15901 100.977029) (end 151.645048 100.977029) (width 0.25) (layer F.Cu) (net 6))
 (segment (start 151.645048 100.977029) (end 154.827029 104.15901) (width 0.25) (layer F.Cu) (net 6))
 (segment (start 127.127029 104.15901) (end 135.127029 104.15901) (width 0.25) (layer F.Cu) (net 6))
 (segment (start 135.127029 104.15901) (end 138.568019 107.6) (width 0.25) (layer F.Cu) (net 6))
 (segment (start 138.568019 107.6) (end 151.386039 107.6) (width 0.25) (layer F.Cu) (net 6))
 (segment (start 151.386039 107.6) (end 154.827029 104.15901) (width 0.25) (layer F.Cu) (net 6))
 (segment (start 154.827029 104.15901) (end 162.827029 104.15901) (width 0.25) (layer F.Cu) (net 6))
 (segment (start 134.40901 79.227029) (end 134.40901 79.09099) (width 0.25) (layer F.Cu) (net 12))
 (segment (start 134.40901 79.09099) (end 136.8 76.7) (width 0.25) (layer F.Cu) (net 12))
 (segment (start 142.36066 76.7) (end 146.151472 72.909188) (width 0.25) (layer F.Cu) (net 12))
 (segment (start 136.8 76.7) (end 142.36066 76.7) (width 0.25) (layer F.Cu) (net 12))
 (segment (start 134.40901 93.727029) (end 135.727029 93.727029) (width 0.25) (layer F.Cu) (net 12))
 (segment (start 144.977029 102.977029) (end 144.977029 104.15901) (width 0.25) (layer F.Cu) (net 12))
 (segment (start 135.727029 93.727029) (end 144.977029 102.977029) (width 0.25) (layer F.Cu) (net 12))
 (segment (start 134.40901 79.227029) (end 134.40901 86.477029) (width 0.25) (layer F.Cu) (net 12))
 (segment (start 134.40901 86.477029) (end 134.40901 93.727029) (width 0.25) (layer F.Cu) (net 12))
 (segment (start 139.90901 93.727029) (end 141.627029 93.727029) (width 0.25) (layer F.Cu) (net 13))
 (segment (start 156.231981 99.2) (end 158.00901 100.977029) (width 0.25) (layer F.Cu) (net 13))
 (segment (start 147.1 99.2) (end 156.231981 99.2) (width 0.25) (layer F.Cu) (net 13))
 (segment (start 141.627029 93.727029) (end 147.1 99.2) (width 0.25) (layer F.Cu) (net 13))
 (segment (start 139.90901 79.227029) (end 140.540738 79.227029) (width 0.25) (layer F.Cu) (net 13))
 (segment (start 140.540738 79.227029) (end 146.505025 73.262742) (width 0.25) (layer F.Cu) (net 13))
 (segment (start 139.90901 79.227029) (end 139.90901 86.477029) (width 0.25) (layer F.Cu) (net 13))
 (segment (start 139.90901 86.477029) (end 139.90901 93.727029) (width 0.25) (layer F.Cu) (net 13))
 (segment (start 145.40901 93.727029) (end 147.127029 93.727029) (width 0.25) (layer F.Cu) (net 14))
 (segment (start 163.631981 98.6) (end 166.00901 100.977029) (width 0.25) (layer F.Cu) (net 14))
 (segment (start 152 98.6) (end 163.631981 98.6) (width 0.25) (layer F.Cu) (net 14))
 (segment (start 147.127029 93.727029) (end 152 98.6) (width 0.25) (layer F.Cu) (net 14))
 (segment (start 147.494975 73.262742) (end 147.494975 73.294975) (width 0.25) (layer F.Cu) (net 14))
 (segment (start 147.494975 73.294975) (end 148.5 74.3) (width 0.25) (layer F.Cu) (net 14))
 (segment (start 148.5 74.3) (end 148.5 76.136039) (width 0.25) (layer F.Cu) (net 14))
 (segment (start 148.5 76.136039) (end 145.40901 79.227029) (width 0.25) (layer F.Cu) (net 14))
 (segment (start 145.40901 79.227029) (end 145.40901 86.477029) (width 0.25) (layer F.Cu) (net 14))
 (segment (start 145.40901 86.477029) (end 145.40901 93.727029) (width 0.25) (layer F.Cu) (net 14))
 (segment (start 150.90901 79.227029) (end 150.90901 76.226775) (width 0.25) (layer F.Cu) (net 15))
 (segment (start 150.9 75.96066) (end 147.848528 72.909188) (width 0.25) (layer F.Cu) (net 15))
 (segment (start 150.9 76.217765) (end 150.9 75.96066) (width 0.25) (layer F.Cu) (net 15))
 (segment (start 150.90901 76.226775) (end 150.9 76.217765) (width 0.25) (layer F.Cu) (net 15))
 (segment (start 150.90901 79.227029) (end 150.90901 86.477029) (width 0.25) (layer F.Cu) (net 15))
 (segment (start 150.90901 86.477029) (end 150.90901 93.727029) (width 0.25) (layer F.Cu) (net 15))
 (segment (start 156.40901 79.227029) (end 154.873476 79.227029) (width 0.25) (layer F.Cu) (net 16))
 (segment (start 154.873476 79.227029) (end 148.202082 72.555635) (width 0.25) (layer F.Cu) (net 16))
 (segment (start 156.40901 79.227029) (end 156.40901 86.477029) (width 0.25) (layer F.Cu) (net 16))
 (segment (start 156.40901 86.477029) (end 156.40901 93.727029) (width 0.25) (layer F.Cu) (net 16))
 (segment (start 161.90901 79.227029) (end 158.727029 79.227029) (width 0.25) (layer F.Cu) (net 17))
 (segment (start 152.653553 76.3) (end 148.555635 72.202082) (width 0.25) (layer F.Cu) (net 17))
 (segment (start 155.8 76.3) (end 152.653553 76.3) (width 0.25) (layer F.Cu) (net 17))
 (segment (start 158.727029 79.227029) (end 155.8 76.3) (width 0.25) (layer F.Cu) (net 17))
 (segment (start 161.90901 79.227029) (end 161.90901 86.477029) (width 0.25) (layer F.Cu) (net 17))
 (segment (start 161.90901 86.477029) (end 161.90901 93.727029) (width 0.25) (layer F.Cu) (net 17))
 (segment (start 167.40901 79.227029) (end 164.227029 79.227029) (width 0.25) (layer F.Cu) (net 18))
 (segment (start 152.489951 75.5) (end 148.873834 71.883883) (width 0.25) (layer F.Cu) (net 18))
 (segment (start 160.5 75.5) (end 152.489951 75.5) (width 0.25) (layer F.Cu) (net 18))
 (segment (start 164.227029 79.227029) (end 160.5 75.5) (width 0.25) (layer F.Cu) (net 18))
 (segment (start 148.873834 71.883883) (end 148.909188 71.848528) (width 0.25) (layer F.Cu) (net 18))
 (segment (start 167.40901 79.227029) (end 167.40901 86.477029) (width 0.25) (layer F.Cu) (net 18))
 (segment (start 167.40901 86.477029) (end 167.40901 93.727029) (width 0.25) (layer F.Cu) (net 18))
 (segment (start 172.90901 79.227029) (end 169.727029 79.227029) (width 0.25) (layer F.Cu) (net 19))
 (segment (start 152.567767 74.8) (end 149.262742 71.494975) (width 0.25) (layer F.Cu) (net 19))
 (segment (start 165.3 74.8) (end 152.567767 74.8) (width 0.25) (layer F.Cu) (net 19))
 (segment (start 169.727029 79.227029) (end 165.3 74.8) (width 0.25) (layer F.Cu) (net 19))
 (segment (start 172.90901 79.227029) (end 172.90901 86.477029) (width 0.25) (layer F.Cu) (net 19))
 (segment (start 172.90901 86.477029) (end 172.90901 93.727029) (width 0.25) (layer F.Cu) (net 19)))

